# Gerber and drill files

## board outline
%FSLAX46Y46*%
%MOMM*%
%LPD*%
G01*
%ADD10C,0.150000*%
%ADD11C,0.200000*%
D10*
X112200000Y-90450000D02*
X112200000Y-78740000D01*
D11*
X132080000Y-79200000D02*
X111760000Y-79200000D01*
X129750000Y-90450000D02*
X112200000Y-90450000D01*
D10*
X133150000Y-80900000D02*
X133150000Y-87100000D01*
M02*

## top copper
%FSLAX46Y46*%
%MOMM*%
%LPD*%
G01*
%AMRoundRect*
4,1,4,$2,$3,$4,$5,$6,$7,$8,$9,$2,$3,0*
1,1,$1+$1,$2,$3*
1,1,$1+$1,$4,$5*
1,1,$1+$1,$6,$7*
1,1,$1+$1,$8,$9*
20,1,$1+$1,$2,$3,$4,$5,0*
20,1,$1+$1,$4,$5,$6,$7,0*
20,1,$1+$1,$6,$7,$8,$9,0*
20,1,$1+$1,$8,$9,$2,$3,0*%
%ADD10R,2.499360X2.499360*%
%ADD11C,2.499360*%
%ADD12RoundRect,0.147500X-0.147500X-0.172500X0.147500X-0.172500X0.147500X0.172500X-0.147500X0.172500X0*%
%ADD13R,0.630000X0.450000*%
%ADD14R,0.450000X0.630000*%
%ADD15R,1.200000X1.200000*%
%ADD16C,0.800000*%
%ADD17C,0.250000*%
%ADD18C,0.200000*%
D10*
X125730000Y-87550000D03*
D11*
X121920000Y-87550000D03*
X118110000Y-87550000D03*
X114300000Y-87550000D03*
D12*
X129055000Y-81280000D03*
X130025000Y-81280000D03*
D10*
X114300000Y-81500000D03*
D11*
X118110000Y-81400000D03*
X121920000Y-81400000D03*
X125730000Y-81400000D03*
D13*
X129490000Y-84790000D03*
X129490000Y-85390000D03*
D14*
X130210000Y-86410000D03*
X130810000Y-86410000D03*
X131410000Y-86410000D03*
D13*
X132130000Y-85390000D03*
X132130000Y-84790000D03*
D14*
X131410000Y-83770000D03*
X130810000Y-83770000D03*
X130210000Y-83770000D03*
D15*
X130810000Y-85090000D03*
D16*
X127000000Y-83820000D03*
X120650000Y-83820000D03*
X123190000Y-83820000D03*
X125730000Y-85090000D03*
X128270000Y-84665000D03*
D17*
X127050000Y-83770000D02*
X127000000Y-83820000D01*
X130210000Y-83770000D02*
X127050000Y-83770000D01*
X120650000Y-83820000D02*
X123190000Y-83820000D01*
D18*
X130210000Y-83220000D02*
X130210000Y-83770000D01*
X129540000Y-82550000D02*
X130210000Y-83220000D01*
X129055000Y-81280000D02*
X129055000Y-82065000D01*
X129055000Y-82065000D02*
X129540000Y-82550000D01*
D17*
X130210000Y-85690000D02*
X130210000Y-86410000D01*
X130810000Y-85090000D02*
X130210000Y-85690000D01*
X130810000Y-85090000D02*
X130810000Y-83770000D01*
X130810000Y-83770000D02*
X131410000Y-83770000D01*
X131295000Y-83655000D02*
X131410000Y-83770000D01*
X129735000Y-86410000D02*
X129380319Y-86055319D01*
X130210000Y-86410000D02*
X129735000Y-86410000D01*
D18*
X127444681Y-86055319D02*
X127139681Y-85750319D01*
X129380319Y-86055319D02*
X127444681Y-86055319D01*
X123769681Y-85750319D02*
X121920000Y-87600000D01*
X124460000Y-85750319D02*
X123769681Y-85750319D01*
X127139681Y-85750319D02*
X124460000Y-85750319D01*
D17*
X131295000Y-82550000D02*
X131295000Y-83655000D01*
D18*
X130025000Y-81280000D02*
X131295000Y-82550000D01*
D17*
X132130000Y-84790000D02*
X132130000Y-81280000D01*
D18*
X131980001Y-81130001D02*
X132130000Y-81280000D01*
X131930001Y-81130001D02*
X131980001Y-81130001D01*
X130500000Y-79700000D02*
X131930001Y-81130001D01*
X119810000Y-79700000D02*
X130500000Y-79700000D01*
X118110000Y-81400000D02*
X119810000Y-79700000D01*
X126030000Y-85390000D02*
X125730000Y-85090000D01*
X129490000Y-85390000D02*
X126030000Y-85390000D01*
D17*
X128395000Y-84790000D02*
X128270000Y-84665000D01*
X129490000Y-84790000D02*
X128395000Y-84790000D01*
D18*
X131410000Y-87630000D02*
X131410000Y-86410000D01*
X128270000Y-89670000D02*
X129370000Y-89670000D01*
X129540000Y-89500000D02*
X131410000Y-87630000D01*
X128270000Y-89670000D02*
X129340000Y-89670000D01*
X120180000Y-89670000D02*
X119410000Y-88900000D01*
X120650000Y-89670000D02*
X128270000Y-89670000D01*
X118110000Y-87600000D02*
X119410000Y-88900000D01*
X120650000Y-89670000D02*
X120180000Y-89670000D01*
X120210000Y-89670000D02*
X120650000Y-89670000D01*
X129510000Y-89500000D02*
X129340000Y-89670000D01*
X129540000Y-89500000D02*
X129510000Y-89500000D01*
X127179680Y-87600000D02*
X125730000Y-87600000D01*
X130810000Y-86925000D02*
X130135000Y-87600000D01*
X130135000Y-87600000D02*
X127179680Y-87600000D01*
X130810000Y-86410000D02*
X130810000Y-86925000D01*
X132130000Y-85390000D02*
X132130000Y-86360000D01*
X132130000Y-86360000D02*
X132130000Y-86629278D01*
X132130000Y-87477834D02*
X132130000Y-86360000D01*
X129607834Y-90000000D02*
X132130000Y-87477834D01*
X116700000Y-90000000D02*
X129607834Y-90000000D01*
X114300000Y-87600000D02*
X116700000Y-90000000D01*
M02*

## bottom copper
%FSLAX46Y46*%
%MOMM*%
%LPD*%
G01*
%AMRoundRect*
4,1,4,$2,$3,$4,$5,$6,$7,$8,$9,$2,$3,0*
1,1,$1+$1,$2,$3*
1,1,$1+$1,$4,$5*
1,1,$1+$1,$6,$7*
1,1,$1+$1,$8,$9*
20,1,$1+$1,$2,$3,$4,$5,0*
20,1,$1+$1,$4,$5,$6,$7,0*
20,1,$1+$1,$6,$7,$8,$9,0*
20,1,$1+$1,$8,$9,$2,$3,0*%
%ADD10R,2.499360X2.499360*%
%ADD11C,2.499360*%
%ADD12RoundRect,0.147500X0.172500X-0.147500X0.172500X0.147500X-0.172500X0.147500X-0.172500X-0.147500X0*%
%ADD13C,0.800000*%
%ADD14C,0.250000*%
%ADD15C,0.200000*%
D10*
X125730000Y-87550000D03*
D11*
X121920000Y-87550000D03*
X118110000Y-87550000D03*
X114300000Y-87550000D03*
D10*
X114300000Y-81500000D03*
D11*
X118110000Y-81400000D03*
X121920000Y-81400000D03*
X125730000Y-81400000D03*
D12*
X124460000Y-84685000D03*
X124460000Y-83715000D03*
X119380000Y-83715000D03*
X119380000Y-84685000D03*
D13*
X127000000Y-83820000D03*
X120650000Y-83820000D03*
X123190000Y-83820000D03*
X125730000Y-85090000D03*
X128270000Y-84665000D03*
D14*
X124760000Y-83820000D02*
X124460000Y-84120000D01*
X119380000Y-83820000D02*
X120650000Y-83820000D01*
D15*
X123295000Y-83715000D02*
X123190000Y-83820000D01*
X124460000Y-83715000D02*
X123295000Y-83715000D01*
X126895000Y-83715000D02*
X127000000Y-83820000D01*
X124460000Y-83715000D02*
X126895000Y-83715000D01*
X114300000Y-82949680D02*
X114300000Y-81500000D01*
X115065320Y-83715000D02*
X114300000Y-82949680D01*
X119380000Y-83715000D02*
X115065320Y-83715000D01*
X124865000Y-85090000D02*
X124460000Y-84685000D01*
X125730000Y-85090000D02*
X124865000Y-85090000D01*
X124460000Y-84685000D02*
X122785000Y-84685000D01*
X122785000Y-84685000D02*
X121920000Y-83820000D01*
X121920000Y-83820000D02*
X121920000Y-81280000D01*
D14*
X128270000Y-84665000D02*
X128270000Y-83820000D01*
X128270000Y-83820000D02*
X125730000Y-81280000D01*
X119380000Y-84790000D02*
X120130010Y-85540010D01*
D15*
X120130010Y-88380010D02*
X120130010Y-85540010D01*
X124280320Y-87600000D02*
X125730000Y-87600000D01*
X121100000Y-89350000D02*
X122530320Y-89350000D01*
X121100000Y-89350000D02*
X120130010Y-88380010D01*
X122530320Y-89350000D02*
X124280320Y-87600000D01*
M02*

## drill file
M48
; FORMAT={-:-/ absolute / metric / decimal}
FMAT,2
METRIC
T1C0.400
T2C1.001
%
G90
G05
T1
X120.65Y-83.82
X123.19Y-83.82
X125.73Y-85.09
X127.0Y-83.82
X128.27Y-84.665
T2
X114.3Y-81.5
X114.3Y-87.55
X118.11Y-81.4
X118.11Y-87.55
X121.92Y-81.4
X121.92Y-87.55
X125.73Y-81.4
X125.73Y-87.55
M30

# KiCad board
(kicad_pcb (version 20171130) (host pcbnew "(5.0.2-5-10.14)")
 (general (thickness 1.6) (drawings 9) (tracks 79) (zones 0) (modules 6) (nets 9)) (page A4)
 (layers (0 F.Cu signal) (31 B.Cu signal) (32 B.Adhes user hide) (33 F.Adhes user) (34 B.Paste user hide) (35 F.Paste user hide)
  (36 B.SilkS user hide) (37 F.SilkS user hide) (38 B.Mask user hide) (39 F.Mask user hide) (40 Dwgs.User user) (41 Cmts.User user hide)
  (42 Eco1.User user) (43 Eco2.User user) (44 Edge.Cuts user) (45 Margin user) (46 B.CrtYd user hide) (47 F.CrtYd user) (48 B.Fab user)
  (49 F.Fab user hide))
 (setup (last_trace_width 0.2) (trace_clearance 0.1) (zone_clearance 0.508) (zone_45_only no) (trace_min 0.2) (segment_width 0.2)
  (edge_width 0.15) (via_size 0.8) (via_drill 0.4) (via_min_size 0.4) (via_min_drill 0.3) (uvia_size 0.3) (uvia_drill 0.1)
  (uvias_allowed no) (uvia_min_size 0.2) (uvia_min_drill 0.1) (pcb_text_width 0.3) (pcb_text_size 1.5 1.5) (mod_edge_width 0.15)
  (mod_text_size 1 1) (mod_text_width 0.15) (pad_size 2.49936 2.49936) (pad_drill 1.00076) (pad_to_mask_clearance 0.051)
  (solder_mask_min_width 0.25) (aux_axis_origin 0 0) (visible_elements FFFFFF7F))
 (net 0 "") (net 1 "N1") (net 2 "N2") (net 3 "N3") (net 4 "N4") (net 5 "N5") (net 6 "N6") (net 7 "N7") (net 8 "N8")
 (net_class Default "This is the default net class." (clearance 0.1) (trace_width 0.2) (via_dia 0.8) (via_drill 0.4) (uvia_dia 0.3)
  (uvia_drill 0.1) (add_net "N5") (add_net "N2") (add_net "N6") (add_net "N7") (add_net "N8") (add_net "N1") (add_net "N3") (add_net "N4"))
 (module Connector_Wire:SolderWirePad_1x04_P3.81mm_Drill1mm (layer F.Cu) (at 125.73 87.55 180)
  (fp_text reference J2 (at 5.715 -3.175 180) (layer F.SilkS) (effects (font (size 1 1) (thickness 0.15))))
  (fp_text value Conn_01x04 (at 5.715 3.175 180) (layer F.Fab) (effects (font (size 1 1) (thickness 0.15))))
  (pad 1 thru_hole rect (at 0 0 180) (size 2.49936 2.49936) (drill 1.00076) (layers *.Cu *.Mask) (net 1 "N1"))
  (pad 2 thru_hole circle (at 3.81 0 180) (size 2.49936 2.49936) (drill 1.00076) (layers *.Cu *.Mask) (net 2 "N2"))
  (pad 3 thru_hole circle (at 7.62 0 180) (size 2.49936 2.49936) (drill 1.00076) (layers *.Cu *.Mask) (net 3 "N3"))
  (pad 4 thru_hole circle (at 11.43 0 180) (size 2.49936 2.49936) (drill 1.00076) (layers *.Cu *.Mask) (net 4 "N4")))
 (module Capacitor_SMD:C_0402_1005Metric (layer F.Cu) (at 129.54 81.28)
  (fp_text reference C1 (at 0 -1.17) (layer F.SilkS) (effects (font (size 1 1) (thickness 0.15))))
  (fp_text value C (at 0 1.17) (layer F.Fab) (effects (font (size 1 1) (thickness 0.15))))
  (pad 1 smd roundrect (at -0.485 0) (size 0.59 0.64) (layers F.Cu F.Paste F.Mask) (roundrect_rratio 0.25) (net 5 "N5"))
  (pad 2 smd roundrect (at 0.485 0) (size 0.59 0.64) (layers F.Cu F.Paste F.Mask) (roundrect_rratio 0.25) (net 2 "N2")))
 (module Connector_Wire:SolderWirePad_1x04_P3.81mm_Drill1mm (layer F.Cu) (at 114.3 81.4)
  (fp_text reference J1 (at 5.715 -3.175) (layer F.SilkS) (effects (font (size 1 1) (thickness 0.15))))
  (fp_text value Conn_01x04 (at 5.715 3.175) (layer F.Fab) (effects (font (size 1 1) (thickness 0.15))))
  (pad 1 thru_hole rect (at 0 0.1) (size 2.49936 2.49936) (drill 1.00076) (layers *.Cu *.Mask) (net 5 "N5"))
  (pad 2 thru_hole circle (at 3.81 0) (size 2.49936 2.49936) (drill 1.00076) (layers *.Cu *.Mask) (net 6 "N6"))
  (pad 3 thru_hole circle (at 7.62 0) (size 2.49936 2.49936) (drill 1.00076) (layers *.Cu *.Mask) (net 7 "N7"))
  (pad 4 thru_hole circle (at 11.43 0) (size 2.49936 2.49936) (drill 1.00076) (layers *.Cu *.Mask) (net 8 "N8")))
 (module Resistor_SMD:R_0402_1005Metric (layer B.Cu) (at 124.46 84.2 90)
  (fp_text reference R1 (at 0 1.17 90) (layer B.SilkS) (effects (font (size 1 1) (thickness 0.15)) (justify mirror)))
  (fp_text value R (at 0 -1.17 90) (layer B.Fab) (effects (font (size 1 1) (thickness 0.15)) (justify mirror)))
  (pad 1 smd roundrect (at -0.485 0 90) (size 0.59 0.64) (layers B.Cu B.Paste B.Mask) (roundrect_rratio 0.25) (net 7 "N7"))
  (pad 2 smd roundrect (at 0.485 0 90) (size 0.59 0.64) (layers B.Cu B.Paste B.Mask) (roundrect_rratio 0.25) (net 5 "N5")))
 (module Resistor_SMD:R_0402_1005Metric (layer B.Cu) (at 119.38 84.2 90)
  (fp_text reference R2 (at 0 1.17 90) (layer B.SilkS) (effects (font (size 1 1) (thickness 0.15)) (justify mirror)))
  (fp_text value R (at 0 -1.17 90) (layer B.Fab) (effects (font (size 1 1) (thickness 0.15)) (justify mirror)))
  (pad 2 smd roundrect (at 0.485 0 90) (size 0.59 0.64) (layers B.Cu B.Paste B.Mask) (roundrect_rratio 0.25) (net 5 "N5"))
  (pad 1 smd roundrect (at -0.485 0 90) (size 0.59 0.64) (layers B.Cu B.Paste B.Mask) (roundrect_rratio 0.25) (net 1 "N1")))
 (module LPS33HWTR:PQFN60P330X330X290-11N (layer F.Cu) (at 130.81 85.09)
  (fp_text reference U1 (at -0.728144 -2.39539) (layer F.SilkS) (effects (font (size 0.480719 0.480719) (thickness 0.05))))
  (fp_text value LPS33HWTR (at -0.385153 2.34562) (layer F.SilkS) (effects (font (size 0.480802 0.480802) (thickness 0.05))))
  (pad 1 smd rect (at -1.32 -0.3) (size 0.63 0.45) (layers F.Cu F.Paste F.Mask) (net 8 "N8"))
  (pad 2 smd rect (at -1.32 0.3) (size 0.63 0.45) (layers F.Cu F.Paste F.Mask) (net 7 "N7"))
  (pad 3 smd rect (at -0.6 1.32 90) (size 0.63 0.45) (layers F.Cu F.Paste F.Mask) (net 2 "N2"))
  (pad 4 smd rect (at 0 1.32 90) (size 0.63 0.45) (layers F.Cu F.Paste F.Mask) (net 1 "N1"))
  (pad 5 smd rect (at 0.6 1.32 90) (size 0.63 0.45) (layers F.Cu F.Paste F.Mask) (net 3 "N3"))
  (pad 6 smd rect (at 1.32 0.3 180) (size 0.63 0.45) (layers F.Cu F.Paste F.Mask) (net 4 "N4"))
  (pad 7 smd rect (at 1.32 -0.3 180) (size 0.63 0.45) (layers F.Cu F.Paste F.Mask) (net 6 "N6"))
  (pad 8 smd rect (at 0.6 -1.32 270) (size 0.63 0.45) (layers F.Cu F.Paste F.Mask) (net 2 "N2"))
  (pad 9 smd rect (at 0 -1.32 270) (size 0.63 0.45) (layers F.Cu F.Paste F.Mask) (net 2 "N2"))
  (pad 10 smd rect (at -0.6 -1.32 270) (size 0.63 0.45) (layers F.Cu F.Paste F.Mask) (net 5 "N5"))
  (pad EP smd rect (at 0 0) (size 1.2 1.2) (layers F.Cu F.Paste F.Mask) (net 2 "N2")))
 (gr_line (start 112.2 90.45) (end 112.2 78.74) (layer Edge.Cuts) (width 0.15))
 (gr_line (start 132.08 79.2) (end 111.76 79.2) (layer Edge.Cuts) (width 0.2))
 (gr_line (start 129.75 90.45) (end 112.2 90.45) (layer Edge.Cuts) (width 0.2))
 (gr_line (start 133.15 80.9) (end 133.15 87.1) (layer Edge.Cuts) (width 0.15))
 (via (at 127 83.82) (size 0.8) (drill 0.4) (layers F.Cu B.Cu) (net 5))
 (segment (start 127.05 83.77) (end 127 83.82) (width 0.25) (layer F.Cu) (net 5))
 (segment (start 130.21 83.77) (end 127.05 83.77) (width 0.25) (layer F.Cu) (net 5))
 (segment (start 124.76 83.82) (end 124.46 84.12) (width 0.25) (layer B.Cu) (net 5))
 (via (at 120.65 83.82) (size 0.8) (drill 0.4) (layers F.Cu B.Cu) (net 5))
 (segment (start 119.38 83.82) (end 120.65 83.82) (width 0.25) (layer B.Cu) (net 5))
 (via (at 123.19 83.82) (size 0.8) (drill 0.4) (layers F.Cu B.Cu) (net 5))
 (segment (start 120.65 83.82) (end 123.19 83.82) (width 0.25) (layer F.Cu) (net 5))
 (segment (start 130.21 83.22) (end 130.21 83.77) (width 0.2) (layer F.Cu) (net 5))
 (segment (start 129.54 82.55) (end 130.21 83.22) (width 0.2) (layer F.Cu) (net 5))
 (segment (start 123.295 83.715) (end 123.19 83.82) (width 0.2) (layer B.Cu) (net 5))
 (segment (start 124.46 83.715) (end 123.295 83.715) (width 0.2) (layer B.Cu) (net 5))
 (segment (start 126.895 83.715) (end 127 83.82) (width 0.2) (layer B.Cu) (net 5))
 (segment (start 124.46 83.715) (end 126.895 83.715) (width 0.2) (layer B.Cu) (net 5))
 (segment (start 114.3 82.94968) (end 114.3 81.5) (width 0.2) (layer B.Cu) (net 5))
 (segment (start 115.06532 83.715) (end 114.3 82.94968) (width 0.2) (layer B.Cu) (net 5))
 (segment (start 119.38 83.715) (end 115.06532 83.715) (width 0.2) (layer B.Cu) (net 5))
 (segment (start 129.055 81.28) (end 129.055 82.065) (width 0.2) (layer F.Cu) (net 5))
 (segment (start 129.055 82.065) (end 129.54 82.55) (width 0.2) (layer F.Cu) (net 5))
 (segment (start 130.21 85.69) (end 130.21 86.41) (width 0.25) (layer F.Cu) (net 2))
 (segment (start 130.81 85.09) (end 130.21 85.69) (width 0.25) (layer F.Cu) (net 2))
 (segment (start 130.81 85.09) (end 130.81 83.77) (width 0.25) (layer F.Cu) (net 2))
 (segment (start 130.81 83.77) (end 131.41 83.77) (width 0.25) (layer F.Cu) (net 2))
 (segment (start 131.295 83.655) (end 131.41 83.77) (width 0.25) (layer F.Cu) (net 2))
 (segment (start 129.735 86.41) (end 129.380319 86.055319) (width 0.25) (layer F.Cu) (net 2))
 (segment (start 130.21 86.41) (end 129.735 86.41) (width 0.25) (layer F.Cu) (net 2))
 (segment (start 127.444681 86.055319) (end 127.139681 85.750319) (width 0.2) (layer F.Cu) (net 2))
 (segment (start 129.380319 86.055319) (end 127.444681 86.055319) (width 0.2) (layer F.Cu) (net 2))
 (segment (start 123.769681 85.750319) (end 121.92 87.6) (width 0.2) (layer F.Cu) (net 2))
 (segment (start 124.46 85.750319) (end 123.769681 85.750319) (width 0.2) (layer F.Cu) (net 2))
 (segment (start 127.139681 85.750319) (end 124.46 85.750319) (width 0.2) (layer F.Cu) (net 2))
 (segment (start 131.295 82.55) (end 131.295 83.655) (width 0.25) (layer F.Cu) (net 2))
 (segment (start 130.025 81.28) (end 131.295 82.55) (width 0.2) (layer F.Cu) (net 2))
 (segment (start 132.13 84.79) (end 132.13 81.28) (width 0.25) (layer F.Cu) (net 6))
 (segment (start 131.980001 81.130001) (end 132.13 81.28) (width 0.2) (layer F.Cu) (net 6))
 (segment (start 131.930001 81.130001) (end 131.980001 81.130001) (width 0.2) (layer F.Cu) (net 6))
 (segment (start 130.5 79.7) (end 131.930001 81.130001) (width 0.2) (layer F.Cu) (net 6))
 (segment (start 119.81 79.7) (end 130.5 79.7) (width 0.2) (layer F.Cu) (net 6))
 (segment (start 118.11 81.4) (end 119.81 79.7) (width 0.2) (layer F.Cu) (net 6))
 (via (at 125.73 85.09) (size 0.8) (drill 0.4) (layers F.Cu B.Cu) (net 7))
 (segment (start 124.865 85.09) (end 124.46 84.685) (width 0.2) (layer B.Cu) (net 7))
 (segment (start 125.73 85.09) (end 124.865 85.09) (width 0.2) (layer B.Cu) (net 7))
 (segment (start 124.46 84.685) (end 122.785 84.685) (width 0.2) (layer B.Cu) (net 7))
 (segment (start 122.785 84.685) (end 121.92 83.82) (width 0.2) (layer B.Cu) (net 7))
 (segment (start 121.92 83.82) (end 121.92 81.28) (width 0.2) (layer B.Cu) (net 7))
 (segment (start 126.03 85.39) (end 125.73 85.09) (width 0.2) (layer F.Cu) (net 7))
 (segment (start 129.49 85.39) (end 126.03 85.39) (width 0.2) (layer F.Cu) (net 7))
 (via (at 128.27 84.665) (size 0.8) (drill 0.4) (layers F.Cu B.Cu) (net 8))
 (segment (start 128.395 84.79) (end 128.27 84.665) (width 0.25) (layer F.Cu) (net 8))
 (segment (start 129.49 84.79) (end 128.395 84.79) (width 0.25) (layer F.Cu) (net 8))
 (segment (start 128.27 84.665) (end 128.27 83.82) (width 0.25) (layer B.Cu) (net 8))
 (segment (start 128.27 83.82) (end 125.73 81.28) (width 0.25) (layer B.Cu) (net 8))
 (segment (start 131.41 87.63) (end 131.41 86.41) (width 0.2) (layer F.Cu) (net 3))
 (segment (start 128.27 89.67) (end 129.37 89.67) (width 0.2) (layer F.Cu) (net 3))
 (segment (start 129.54 89.5) (end 131.41 87.63) (width 0.2) (layer F.Cu) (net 3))
 (segment (start 128.27 89.67) (end 129.34 89.67) (width 0.2) (layer F.Cu) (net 3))
 (segment (start 120.18 89.67) (end 119.41 88.9) (width 0.2) (layer F.Cu) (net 3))
 (segment (start 120.65 89.67) (end 128.27 89.67) (width 0.2) (layer F.Cu) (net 3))
 (segment (start 118.11 87.6) (end 119.41 88.9) (width 0.2) (layer F.Cu) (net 3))
 (segment (start 120.65 89.67) (end 120.18 89.67) (width 0.2) (layer F.Cu) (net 3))
 (segment (start 120.21 89.67) (end 120.65 89.67) (width 0.2) (layer F.Cu) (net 3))
 (segment (start 129.51 89.5) (end 129.34 89.67) (width 0.2) (layer F.Cu) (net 3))
 (segment (start 129.54 89.5) (end 129.51 89.5) (width 0.2) (layer F.Cu) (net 3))
 (segment (start 119.38 84.79) (end 120.13001 85.54001) (width 0.25) (layer B.Cu) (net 1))
 (segment (start 127.17968 87.6) (end 125.73 87.6) (width 0.2) (layer F.Cu) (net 1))
 (segment (start 130.81 86.925) (end 130.135 87.6) (width 0.2) (layer F.Cu) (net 1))
 (segment (start 130.135 87.6) (end 127.17968 87.6) (width 0.2) (layer F.Cu) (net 1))
 (segment (start 130.81 86.41) (end 130.81 86.925) (width 0.2) (layer F.Cu) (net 1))
 (segment (start 120.13001 88.38001) (end 120.13001 85.54001) (width 0.2) (layer B.Cu) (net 1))
 (segment (start 124.28032 87.6) (end 125.73 87.6) (width 0.2) (layer B.Cu) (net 1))
 (segment (start 121.1 89.35) (end 122.53032 89.35) (width 0.2) (layer B.Cu) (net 1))
 (segment (start 121.1 89.35) (end 120.13001 88.38001) (width 0.2) (layer B.Cu) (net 1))
 (segment (start 122.53032 89.35) (end 124.28032 87.6) (width 0.2) (layer B.Cu) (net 1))
 (segment (start 132.13 85.39) (end 132.13 86.36) (width 0.2) (layer F.Cu) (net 4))
 (segment (start 132.13 86.36) (end 132.13 86.629278) (width 0.2) (layer F.Cu) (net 4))
 (segment (start 132.13 87.477834) (end 132.13 86.36) (width 0.2) (layer F.Cu) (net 4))
 (segment (start 129.607834 90) (end 132.13 87.477834) (width 0.2) (layer F.Cu) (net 4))
 (segment (start 116.7 90) (end 129.607834 90) (width 0.2) (layer F.Cu) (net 4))
 (segment (start 114.3 87.6) (end 116.7 90) (width 0.2) (layer F.Cu) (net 4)))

